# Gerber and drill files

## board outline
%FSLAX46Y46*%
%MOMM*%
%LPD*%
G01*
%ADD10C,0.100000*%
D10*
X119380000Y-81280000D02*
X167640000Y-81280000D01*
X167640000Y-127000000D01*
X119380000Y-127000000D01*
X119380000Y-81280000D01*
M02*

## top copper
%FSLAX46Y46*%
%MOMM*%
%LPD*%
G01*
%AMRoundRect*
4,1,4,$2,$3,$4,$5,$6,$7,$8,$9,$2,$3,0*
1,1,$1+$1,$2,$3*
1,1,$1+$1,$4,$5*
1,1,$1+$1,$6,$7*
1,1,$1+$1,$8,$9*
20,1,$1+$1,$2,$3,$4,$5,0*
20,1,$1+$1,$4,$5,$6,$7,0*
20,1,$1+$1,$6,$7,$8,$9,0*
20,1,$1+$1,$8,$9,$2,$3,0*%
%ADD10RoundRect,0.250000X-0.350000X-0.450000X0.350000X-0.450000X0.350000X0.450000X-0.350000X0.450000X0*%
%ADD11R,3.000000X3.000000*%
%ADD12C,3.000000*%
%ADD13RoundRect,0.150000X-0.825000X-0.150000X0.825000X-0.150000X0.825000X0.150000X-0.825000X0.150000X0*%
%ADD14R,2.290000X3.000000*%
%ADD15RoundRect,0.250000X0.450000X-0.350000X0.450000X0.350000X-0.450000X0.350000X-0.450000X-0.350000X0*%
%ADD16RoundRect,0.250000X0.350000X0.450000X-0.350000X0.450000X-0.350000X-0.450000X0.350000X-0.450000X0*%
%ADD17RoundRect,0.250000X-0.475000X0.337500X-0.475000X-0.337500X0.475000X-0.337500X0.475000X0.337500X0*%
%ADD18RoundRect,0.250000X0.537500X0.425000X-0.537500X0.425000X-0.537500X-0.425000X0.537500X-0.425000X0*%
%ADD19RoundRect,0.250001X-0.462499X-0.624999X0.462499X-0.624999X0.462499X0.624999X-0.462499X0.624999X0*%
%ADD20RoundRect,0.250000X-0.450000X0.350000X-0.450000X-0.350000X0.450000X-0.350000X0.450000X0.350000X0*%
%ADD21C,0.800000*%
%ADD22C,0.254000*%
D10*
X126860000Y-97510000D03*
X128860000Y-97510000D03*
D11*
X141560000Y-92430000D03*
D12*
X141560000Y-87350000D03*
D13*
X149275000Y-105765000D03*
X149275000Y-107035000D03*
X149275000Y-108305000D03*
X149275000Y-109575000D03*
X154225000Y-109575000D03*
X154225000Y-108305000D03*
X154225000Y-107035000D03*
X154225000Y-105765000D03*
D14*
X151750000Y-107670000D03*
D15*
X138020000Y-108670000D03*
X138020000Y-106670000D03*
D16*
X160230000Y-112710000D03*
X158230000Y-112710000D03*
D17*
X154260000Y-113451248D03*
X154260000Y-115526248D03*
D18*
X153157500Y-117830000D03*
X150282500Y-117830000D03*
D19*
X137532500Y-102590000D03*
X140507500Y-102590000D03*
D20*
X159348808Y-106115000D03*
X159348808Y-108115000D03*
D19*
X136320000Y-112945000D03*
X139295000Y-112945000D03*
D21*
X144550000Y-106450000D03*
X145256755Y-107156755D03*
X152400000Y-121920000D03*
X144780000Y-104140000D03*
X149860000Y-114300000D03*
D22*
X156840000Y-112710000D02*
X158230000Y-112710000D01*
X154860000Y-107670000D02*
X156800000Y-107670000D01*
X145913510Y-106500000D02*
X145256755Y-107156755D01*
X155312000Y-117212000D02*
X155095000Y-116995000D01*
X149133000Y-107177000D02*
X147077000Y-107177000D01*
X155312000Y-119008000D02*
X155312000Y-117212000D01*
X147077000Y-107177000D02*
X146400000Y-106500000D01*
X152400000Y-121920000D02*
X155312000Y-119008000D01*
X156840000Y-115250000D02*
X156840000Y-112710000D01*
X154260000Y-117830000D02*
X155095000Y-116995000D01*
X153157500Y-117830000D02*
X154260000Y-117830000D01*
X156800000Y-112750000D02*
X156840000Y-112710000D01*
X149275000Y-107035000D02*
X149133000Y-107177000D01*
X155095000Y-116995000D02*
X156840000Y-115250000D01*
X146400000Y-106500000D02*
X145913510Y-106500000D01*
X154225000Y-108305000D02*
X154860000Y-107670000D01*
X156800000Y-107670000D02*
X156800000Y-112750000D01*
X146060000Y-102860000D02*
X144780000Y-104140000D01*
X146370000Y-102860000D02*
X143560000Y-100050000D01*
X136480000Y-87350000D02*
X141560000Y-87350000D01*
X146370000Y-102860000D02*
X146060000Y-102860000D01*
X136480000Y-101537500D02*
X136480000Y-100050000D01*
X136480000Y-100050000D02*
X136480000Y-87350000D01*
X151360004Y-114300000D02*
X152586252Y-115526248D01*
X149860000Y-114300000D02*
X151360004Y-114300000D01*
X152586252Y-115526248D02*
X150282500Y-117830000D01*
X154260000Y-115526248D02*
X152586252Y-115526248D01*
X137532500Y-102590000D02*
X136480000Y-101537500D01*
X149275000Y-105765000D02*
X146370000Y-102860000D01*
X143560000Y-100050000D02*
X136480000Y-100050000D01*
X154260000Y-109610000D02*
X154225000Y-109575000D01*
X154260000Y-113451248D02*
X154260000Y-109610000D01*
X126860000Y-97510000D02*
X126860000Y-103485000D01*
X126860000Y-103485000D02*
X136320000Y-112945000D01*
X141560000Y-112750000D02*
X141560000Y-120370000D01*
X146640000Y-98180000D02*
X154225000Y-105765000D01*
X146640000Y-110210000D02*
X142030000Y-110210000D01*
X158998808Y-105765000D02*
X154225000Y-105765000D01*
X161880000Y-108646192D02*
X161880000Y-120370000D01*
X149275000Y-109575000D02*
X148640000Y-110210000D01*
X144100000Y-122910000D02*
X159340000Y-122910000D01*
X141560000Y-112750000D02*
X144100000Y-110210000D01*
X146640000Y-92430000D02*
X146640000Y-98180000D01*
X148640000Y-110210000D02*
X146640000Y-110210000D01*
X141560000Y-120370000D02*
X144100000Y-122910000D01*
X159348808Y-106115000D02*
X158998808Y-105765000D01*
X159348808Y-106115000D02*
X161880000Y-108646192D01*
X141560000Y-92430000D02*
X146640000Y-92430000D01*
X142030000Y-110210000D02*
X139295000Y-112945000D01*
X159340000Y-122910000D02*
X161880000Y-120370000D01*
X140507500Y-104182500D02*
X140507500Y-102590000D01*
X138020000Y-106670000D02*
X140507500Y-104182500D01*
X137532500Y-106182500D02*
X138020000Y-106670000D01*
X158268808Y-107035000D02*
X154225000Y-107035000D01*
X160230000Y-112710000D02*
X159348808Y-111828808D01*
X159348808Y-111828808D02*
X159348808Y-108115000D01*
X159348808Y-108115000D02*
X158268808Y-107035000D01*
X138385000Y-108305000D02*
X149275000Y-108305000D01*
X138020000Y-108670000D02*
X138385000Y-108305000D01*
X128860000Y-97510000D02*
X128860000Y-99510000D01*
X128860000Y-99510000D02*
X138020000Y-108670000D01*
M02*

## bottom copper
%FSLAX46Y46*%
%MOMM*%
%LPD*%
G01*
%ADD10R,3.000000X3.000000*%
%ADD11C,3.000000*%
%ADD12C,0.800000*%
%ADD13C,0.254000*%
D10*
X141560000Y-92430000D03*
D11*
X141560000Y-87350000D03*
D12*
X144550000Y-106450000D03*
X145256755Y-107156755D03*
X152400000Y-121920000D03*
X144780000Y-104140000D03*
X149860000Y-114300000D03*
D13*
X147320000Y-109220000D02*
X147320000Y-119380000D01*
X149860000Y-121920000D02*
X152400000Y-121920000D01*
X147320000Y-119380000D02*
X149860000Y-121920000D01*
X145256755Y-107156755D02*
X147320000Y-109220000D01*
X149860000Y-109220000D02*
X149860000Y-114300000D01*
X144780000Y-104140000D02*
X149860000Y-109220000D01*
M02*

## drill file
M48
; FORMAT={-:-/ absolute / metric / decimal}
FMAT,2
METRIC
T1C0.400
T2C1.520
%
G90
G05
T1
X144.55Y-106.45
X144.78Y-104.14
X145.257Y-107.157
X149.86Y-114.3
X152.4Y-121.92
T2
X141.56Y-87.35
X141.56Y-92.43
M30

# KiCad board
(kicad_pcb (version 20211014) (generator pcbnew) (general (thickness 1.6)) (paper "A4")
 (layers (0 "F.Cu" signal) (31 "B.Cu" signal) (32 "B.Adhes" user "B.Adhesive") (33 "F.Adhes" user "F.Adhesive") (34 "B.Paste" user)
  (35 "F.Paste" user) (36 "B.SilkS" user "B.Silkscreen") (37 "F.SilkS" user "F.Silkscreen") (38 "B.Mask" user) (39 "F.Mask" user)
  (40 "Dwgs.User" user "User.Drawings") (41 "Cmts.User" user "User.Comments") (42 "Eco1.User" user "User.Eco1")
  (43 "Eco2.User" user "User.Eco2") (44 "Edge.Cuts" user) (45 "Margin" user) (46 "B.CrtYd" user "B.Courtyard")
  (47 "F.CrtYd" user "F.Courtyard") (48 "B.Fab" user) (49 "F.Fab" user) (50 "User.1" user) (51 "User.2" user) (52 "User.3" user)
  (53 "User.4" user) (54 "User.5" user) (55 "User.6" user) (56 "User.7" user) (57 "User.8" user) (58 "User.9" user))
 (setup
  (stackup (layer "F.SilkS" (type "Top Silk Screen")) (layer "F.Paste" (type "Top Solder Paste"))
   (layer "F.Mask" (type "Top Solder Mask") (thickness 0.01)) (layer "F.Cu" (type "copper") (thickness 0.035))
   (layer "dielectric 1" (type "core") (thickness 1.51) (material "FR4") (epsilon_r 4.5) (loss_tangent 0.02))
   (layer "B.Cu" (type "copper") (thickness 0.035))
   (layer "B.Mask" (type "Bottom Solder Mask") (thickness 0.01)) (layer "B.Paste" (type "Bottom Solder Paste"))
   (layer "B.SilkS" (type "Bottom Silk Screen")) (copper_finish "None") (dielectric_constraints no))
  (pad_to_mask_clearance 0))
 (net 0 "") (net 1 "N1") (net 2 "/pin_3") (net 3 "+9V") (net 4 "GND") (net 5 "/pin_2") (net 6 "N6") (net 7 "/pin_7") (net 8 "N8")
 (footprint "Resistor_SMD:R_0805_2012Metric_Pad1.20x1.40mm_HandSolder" (layer "F.Cu") (at 127.86 97.51)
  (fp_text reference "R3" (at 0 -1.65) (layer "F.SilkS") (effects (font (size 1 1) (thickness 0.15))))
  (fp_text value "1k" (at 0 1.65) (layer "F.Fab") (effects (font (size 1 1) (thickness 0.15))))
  (pad "1" smd roundrect (at -1 0) (size 1.2 1.4) (layers "F.Cu" "F.Paste" "F.Mask") (roundrect_rratio 0.2083333333) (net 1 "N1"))
  (pad "2" smd roundrect (at 1 0) (size 1.2 1.4) (layers "F.Cu" "F.Paste" "F.Mask") (roundrect_rratio 0.2083333333) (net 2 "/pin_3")))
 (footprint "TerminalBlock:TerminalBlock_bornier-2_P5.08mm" (layer "F.Cu") (at 141.56 92.43 90)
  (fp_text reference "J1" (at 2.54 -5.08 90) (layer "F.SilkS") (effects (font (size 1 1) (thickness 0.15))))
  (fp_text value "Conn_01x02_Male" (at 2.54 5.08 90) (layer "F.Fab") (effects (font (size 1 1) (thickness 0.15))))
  (pad "1" thru_hole rect (at 0 0 90) (size 3 3) (drill 1.52) (layers *.Cu *.Mask) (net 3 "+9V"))
  (pad "2" thru_hole circle (at 5.08 0 90) (size 3 3) (drill 1.52) (layers *.Cu *.Mask) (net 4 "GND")))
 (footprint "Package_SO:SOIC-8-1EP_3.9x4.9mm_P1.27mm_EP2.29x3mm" (layer "F.Cu") (at 151.75 107.67)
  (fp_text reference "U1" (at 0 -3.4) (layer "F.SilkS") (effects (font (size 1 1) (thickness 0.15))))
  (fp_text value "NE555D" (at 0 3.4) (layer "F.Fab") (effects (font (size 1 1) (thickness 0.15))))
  (pad "" smd roundrect (at 0.57 -0.75) (size 0.92 1.21) (layers "F.Paste") (roundrect_rratio 0.25))
  (pad "" smd roundrect (at -0.57 -0.75) (size 0.92 1.21) (layers "F.Paste") (roundrect_rratio 0.25))
  (pad "" smd roundrect (at 0.57 0.75) (size 0.92 1.21) (layers "F.Paste") (roundrect_rratio 0.25))
  (pad "" smd roundrect (at -0.57 0.75) (size 0.92 1.21) (layers "F.Paste") (roundrect_rratio 0.25))
  (pad "1" smd roundrect (at -2.475 -1.905) (size 1.95 0.6) (layers "F.Cu" "F.Paste" "F.Mask") (roundrect_rratio 0.25) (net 4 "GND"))
  (pad "2" smd roundrect (at -2.475 -0.635) (size 1.95 0.6) (layers "F.Cu" "F.Paste" "F.Mask") (roundrect_rratio 0.25) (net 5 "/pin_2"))
  (pad "3" smd roundrect (at -2.475 0.635) (size 1.95 0.6) (layers "F.Cu" "F.Paste" "F.Mask") (roundrect_rratio 0.25) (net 2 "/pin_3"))
  (pad "4" smd roundrect (at -2.475 1.905) (size 1.95 0.6) (layers "F.Cu" "F.Paste" "F.Mask") (roundrect_rratio 0.25) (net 3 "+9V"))
  (pad "5" smd roundrect (at 2.475 1.905) (size 1.95 0.6) (layers "F.Cu" "F.Paste" "F.Mask") (roundrect_rratio 0.25) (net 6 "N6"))
  (pad "6" smd roundrect (at 2.475 0.635) (size 1.95 0.6) (layers "F.Cu" "F.Paste" "F.Mask") (roundrect_rratio 0.25) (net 5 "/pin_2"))
  (pad "7" smd roundrect (at 2.475 -0.635) (size 1.95 0.6) (layers "F.Cu" "F.Paste" "F.Mask") (roundrect_rratio 0.25) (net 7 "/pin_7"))
  (pad "8" smd roundrect (at 2.475 -1.905) (size 1.95 0.6) (layers "F.Cu" "F.Paste" "F.Mask") (roundrect_rratio 0.25) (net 3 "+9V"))
  (pad "9" smd rect (at 0 0) (size 2.29 3) (layers "F.Cu" "F.Mask")))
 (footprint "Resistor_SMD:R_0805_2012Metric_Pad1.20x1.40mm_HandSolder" (layer "F.Cu") (at 138.02 107.67 90)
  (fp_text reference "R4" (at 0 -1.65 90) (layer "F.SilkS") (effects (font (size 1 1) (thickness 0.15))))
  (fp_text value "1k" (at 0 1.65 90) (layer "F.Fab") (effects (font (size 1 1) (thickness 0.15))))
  (pad "1" smd roundrect (at -1 0 90) (size 1.2 1.4) (layers "F.Cu" "F.Paste" "F.Mask") (roundrect_rratio 0.2083333333) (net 2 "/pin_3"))
  (pad "2" smd roundrect (at 1 0 90) (size 1.2 1.4) (layers "F.Cu" "F.Paste" "F.Mask") (roundrect_rratio 0.2083333333) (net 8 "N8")))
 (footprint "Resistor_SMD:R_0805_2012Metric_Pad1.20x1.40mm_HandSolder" (layer "F.Cu") (at 159.23 112.71 180)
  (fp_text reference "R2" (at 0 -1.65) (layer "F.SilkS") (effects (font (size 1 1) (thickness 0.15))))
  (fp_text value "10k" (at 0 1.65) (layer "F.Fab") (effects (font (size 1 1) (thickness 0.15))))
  (pad "1" smd roundrect (at -1 0 180) (size 1.2 1.4) (layers "F.Cu" "F.Paste" "F.Mask") (roundrect_rratio 0.2083333333) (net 7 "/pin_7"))
  (pad "2" smd roundrect (at 1 0 180) (size 1.2 1.4) (layers "F.Cu" "F.Paste" "F.Mask") (roundrect_rratio 0.2083333333) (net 5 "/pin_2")))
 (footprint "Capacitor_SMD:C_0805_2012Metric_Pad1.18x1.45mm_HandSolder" (layer "F.Cu") (at 154.26 114.488748 -90)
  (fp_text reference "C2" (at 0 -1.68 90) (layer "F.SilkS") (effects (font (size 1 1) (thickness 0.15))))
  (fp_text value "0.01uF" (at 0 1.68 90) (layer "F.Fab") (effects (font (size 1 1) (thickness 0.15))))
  (pad "1" smd roundrect (at -1.0375 0 270) (size 1.175 1.45) (layers "F.Cu" "F.Paste" "F.Mask") (roundrect_rratio 0.2127659574)
   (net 6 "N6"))
  (pad "2" smd roundrect (at 1.0375 0 270) (size 1.175 1.45) (layers "F.Cu" "F.Paste" "F.Mask") (roundrect_rratio 0.2127659574)
   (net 4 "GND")))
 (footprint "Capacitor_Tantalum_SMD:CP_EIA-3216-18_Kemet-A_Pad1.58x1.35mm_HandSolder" (layer "F.Cu") (at 151.72 117.83 180)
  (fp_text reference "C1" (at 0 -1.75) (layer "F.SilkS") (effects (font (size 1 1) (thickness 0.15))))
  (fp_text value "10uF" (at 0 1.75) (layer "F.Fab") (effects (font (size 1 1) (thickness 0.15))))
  (pad "1" smd roundrect (at -1.4375 0 180) (size 1.575 1.35) (layers "F.Cu" "F.Paste" "F.Mask") (roundrect_rratio 0.1851851852)
   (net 5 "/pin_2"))
  (pad "2" smd roundrect (at 1.4375 0 180) (size 1.575 1.35) (layers "F.Cu" "F.Paste" "F.Mask") (roundrect_rratio 0.1851851852)
   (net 4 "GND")))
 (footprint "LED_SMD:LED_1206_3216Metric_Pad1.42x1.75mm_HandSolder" (layer "F.Cu") (at 139.02 102.59)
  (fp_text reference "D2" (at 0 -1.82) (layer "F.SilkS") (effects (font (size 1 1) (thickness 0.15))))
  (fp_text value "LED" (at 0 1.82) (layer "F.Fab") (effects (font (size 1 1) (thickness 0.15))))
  (pad "1" smd roundrect (at -1.4875 0) (size 1.425 1.75) (layers "F.Cu" "F.Paste" "F.Mask") (roundrect_rratio 0.1754392982) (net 4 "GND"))
  (pad "2" smd roundrect (at 1.4875 0) (size 1.425 1.75) (layers "F.Cu" "F.Paste" "F.Mask") (roundrect_rratio 0.1754392982) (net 8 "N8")))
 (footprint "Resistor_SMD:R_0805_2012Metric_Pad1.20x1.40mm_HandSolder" (layer "F.Cu") (at 159.348808 107.115 -90)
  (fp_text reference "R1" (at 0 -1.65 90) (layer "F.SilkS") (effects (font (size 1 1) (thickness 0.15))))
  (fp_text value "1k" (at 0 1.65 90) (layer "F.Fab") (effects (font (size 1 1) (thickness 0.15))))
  (pad "1" smd roundrect (at -1 0 270) (size 1.2 1.4) (layers "F.Cu" "F.Paste" "F.Mask") (roundrect_rratio 0.2083333333) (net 3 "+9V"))
  (pad "2" smd roundrect (at 1 0 270) (size 1.2 1.4) (layers "F.Cu" "F.Paste" "F.Mask") (roundrect_rratio 0.2083333333) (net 7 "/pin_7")))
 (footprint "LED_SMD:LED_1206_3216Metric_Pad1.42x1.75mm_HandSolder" (layer "F.Cu") (at 137.8075 112.945)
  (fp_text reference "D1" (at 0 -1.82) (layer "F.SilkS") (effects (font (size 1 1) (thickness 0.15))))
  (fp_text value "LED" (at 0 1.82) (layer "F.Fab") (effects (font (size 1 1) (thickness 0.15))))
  (pad "1" smd roundrect (at -1.4875 0) (size 1.425 1.75) (layers "F.Cu" "F.Paste" "F.Mask") (roundrect_rratio 0.1754392982) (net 1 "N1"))
  (pad "2" smd roundrect (at 1.4875 0) (size 1.425 1.75) (layers "F.Cu" "F.Paste" "F.Mask") (roundrect_rratio 0.1754392982) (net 3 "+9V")))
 (gr_rect (start 119.38 81.28) (end 167.64 127) (layer "Edge.Cuts") (width 0.1) (fill none))
 (via (at 144.55 106.45) (size 0.8) (drill 0.4) (layers "F.Cu" "B.Cu") (free) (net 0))
 (segment (start 156.84 112.71) (end 158.23 112.71) (width 0.254) (layer "F.Cu") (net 5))
 (segment (start 154.86 107.67) (end 156.8 107.67) (width 0.254) (layer "F.Cu") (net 5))
 (segment (start 145.91351 106.5) (end 145.256755 107.156755) (width 0.254) (layer "F.Cu") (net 5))
 (segment (start 155.312 117.212) (end 155.095 116.995) (width 0.254) (layer "F.Cu") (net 5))
 (segment (start 149.133 107.177) (end 147.077 107.177) (width 0.254) (layer "F.Cu") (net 5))
 (segment (start 155.312 119.008) (end 155.312 117.212) (width 0.254) (layer "F.Cu") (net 5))
 (segment (start 147.077 107.177) (end 146.4 106.5) (width 0.254) (layer "F.Cu") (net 5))
 (segment (start 152.4 121.92) (end 155.312 119.008) (width 0.254) (layer "F.Cu") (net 5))
 (segment (start 156.84 115.25) (end 156.84 112.71) (width 0.254) (layer "F.Cu") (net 5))
 (segment (start 154.26 117.83) (end 155.095 116.995) (width 0.254) (layer "F.Cu") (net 5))
 (segment (start 153.1575 117.83) (end 154.26 117.83) (width 0.254) (layer "F.Cu") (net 5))
 (segment (start 156.8 112.75) (end 156.84 112.71) (width 0.254) (layer "F.Cu") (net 5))
 (segment (start 149.275 107.035) (end 149.133 107.177) (width 0.254) (layer "F.Cu") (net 5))
 (segment (start 155.095 116.995) (end 156.84 115.25) (width 0.254) (layer "F.Cu") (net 5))
 (segment (start 146.4 106.5) (end 145.91351 106.5) (width 0.254) (layer "F.Cu") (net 5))
 (segment (start 154.225 108.305) (end 154.86 107.67) (width 0.254) (layer "F.Cu") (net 5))
 (segment (start 156.8 107.67) (end 156.8 112.75) (width 0.254) (layer "F.Cu") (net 5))
 (via (at 145.256755 107.156755) (size 0.8) (drill 0.4) (layers "F.Cu" "B.Cu") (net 5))
 (via (at 152.4 121.92) (size 0.8) (drill 0.4) (layers "F.Cu" "B.Cu") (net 5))
 (segment (start 147.32 109.22) (end 147.32 119.38) (width 0.254) (layer "B.Cu") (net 5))
 (segment (start 149.86 121.92) (end 152.4 121.92) (width 0.254) (layer "B.Cu") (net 5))
 (segment (start 147.32 119.38) (end 149.86 121.92) (width 0.254) (layer "B.Cu") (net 5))
 (segment (start 145.256755 107.156755) (end 147.32 109.22) (width 0.254) (layer "B.Cu") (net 5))
 (segment (start 146.06 102.86) (end 144.78 104.14) (width 0.254) (layer "F.Cu") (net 4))
 (segment (start 146.37 102.86) (end 143.56 100.05) (width 0.254) (layer "F.Cu") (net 4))
 (segment (start 136.48 87.35) (end 141.56 87.35) (width 0.254) (layer "F.Cu") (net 4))
 (segment (start 146.37 102.86) (end 146.06 102.86) (width 0.254) (layer "F.Cu") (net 4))
 (segment (start 136.48 101.5375) (end 136.48 100.05) (width 0.254) (layer "F.Cu") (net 4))
 (segment (start 136.48 100.05) (end 136.48 87.35) (width 0.254) (layer "F.Cu") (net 4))
 (segment (start 151.360004 114.3) (end 152.586252 115.526248) (width 0.254) (layer "F.Cu") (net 4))
 (segment (start 149.86 114.3) (end 151.360004 114.3) (width 0.254) (layer "F.Cu") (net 4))
 (segment (start 152.586252 115.526248) (end 150.2825 117.83) (width 0.254) (layer "F.Cu") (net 4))
 (segment (start 154.26 115.526248) (end 152.586252 115.526248) (width 0.254) (layer "F.Cu") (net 4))
 (segment (start 137.5325 102.59) (end 136.48 101.5375) (width 0.254) (layer "F.Cu") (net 4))
 (segment (start 149.275 105.765) (end 146.37 102.86) (width 0.254) (layer "F.Cu") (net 4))
 (segment (start 143.56 100.05) (end 136.48 100.05) (width 0.254) (layer "F.Cu") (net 4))
 (via (at 144.78 104.14) (size 0.8) (drill 0.4) (layers "F.Cu" "B.Cu") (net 4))
 (via (at 149.86 114.3) (size 0.8) (drill 0.4) (layers "F.Cu" "B.Cu") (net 4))
 (segment (start 149.86 109.22) (end 149.86 114.3) (width 0.254) (layer "B.Cu") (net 4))
 (segment (start 144.78 104.14) (end 149.86 109.22) (width 0.254) (layer "B.Cu") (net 4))
 (segment (start 154.26 109.61) (end 154.225 109.575) (width 0.254) (layer "F.Cu") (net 6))
 (segment (start 154.26 113.451248) (end 154.26 109.61) (width 0.254) (layer "F.Cu") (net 6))
 (segment (start 126.86 97.51) (end 126.86 103.485) (width 0.254) (layer "F.Cu") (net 1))
 (segment (start 126.86 103.485) (end 136.32 112.945) (width 0.254) (layer "F.Cu") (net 1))
 (segment (start 141.56 112.75) (end 141.56 120.37) (width 0.254) (layer "F.Cu") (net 3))
 (segment (start 146.64 98.18) (end 154.225 105.765) (width 0.254) (layer "F.Cu") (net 3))
 (segment (start 146.64 110.21) (end 142.03 110.21) (width 0.254) (layer "F.Cu") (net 3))
 (segment (start 158.998808 105.765) (end 154.225 105.765) (width 0.254) (layer "F.Cu") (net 3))
 (segment (start 161.88 108.646192) (end 161.88 120.37) (width 0.254) (layer "F.Cu") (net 3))
 (segment (start 149.275 109.575) (end 148.64 110.21) (width 0.254) (layer "F.Cu") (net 3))
 (segment (start 144.1 122.91) (end 159.34 122.91) (width 0.254) (layer "F.Cu") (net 3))
 (segment (start 141.56 112.75) (end 144.1 110.21) (width 0.254) (layer "F.Cu") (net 3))
 (segment (start 146.64 92.43) (end 146.64 98.18) (width 0.254) (layer "F.Cu") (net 3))
 (segment (start 148.64 110.21) (end 146.64 110.21) (width 0.254) (layer "F.Cu") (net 3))
 (segment (start 141.56 120.37) (end 144.1 122.91) (width 0.254) (layer "F.Cu") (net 3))
 (segment (start 159.348808 106.115) (end 158.998808 105.765) (width 0.254) (layer "F.Cu") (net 3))
 (segment (start 159.348808 106.115) (end 161.88 108.646192) (width 0.254) (layer "F.Cu") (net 3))
 (segment (start 141.56 92.43) (end 146.64 92.43) (width 0.254) (layer "F.Cu") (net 3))
 (segment (start 142.03 110.21) (end 139.295 112.945) (width 0.254) (layer "F.Cu") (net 3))
 (segment (start 159.34 122.91) (end 161.88 120.37) (width 0.254) (layer "F.Cu") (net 3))
 (segment (start 140.5075 104.1825) (end 140.5075 102.59) (width 0.254) (layer "F.Cu") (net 8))
 (segment (start 138.02 106.67) (end 140.5075 104.1825) (width 0.254) (layer "F.Cu") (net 8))
 (segment (start 137.5325 106.1825) (end 138.02 106.67) (width 0.254) (layer "F.Cu") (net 8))
 (segment (start 158.268808 107.035) (end 154.225 107.035) (width 0.254) (layer "F.Cu") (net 7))
 (segment (start 160.23 112.71) (end 159.348808 111.828808) (width 0.254) (layer "F.Cu") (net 7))
 (segment (start 159.348808 111.828808) (end 159.348808 108.115) (width 0.254) (layer "F.Cu") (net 7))
 (segment (start 159.348808 108.115) (end 158.268808 107.035) (width 0.254) (layer "F.Cu") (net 7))
 (segment (start 138.385 108.305) (end 149.275 108.305) (width 0.254) (layer "F.Cu") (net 2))
 (segment (start 138.02 108.67) (end 138.385 108.305) (width 0.254) (layer "F.Cu") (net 2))
 (segment (start 128.86 97.51) (end 128.86 99.51) (width 0.254) (layer "F.Cu") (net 2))
 (segment (start 128.86 99.51) (end 138.02 108.67) (width 0.254) (layer "F.Cu") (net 2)))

